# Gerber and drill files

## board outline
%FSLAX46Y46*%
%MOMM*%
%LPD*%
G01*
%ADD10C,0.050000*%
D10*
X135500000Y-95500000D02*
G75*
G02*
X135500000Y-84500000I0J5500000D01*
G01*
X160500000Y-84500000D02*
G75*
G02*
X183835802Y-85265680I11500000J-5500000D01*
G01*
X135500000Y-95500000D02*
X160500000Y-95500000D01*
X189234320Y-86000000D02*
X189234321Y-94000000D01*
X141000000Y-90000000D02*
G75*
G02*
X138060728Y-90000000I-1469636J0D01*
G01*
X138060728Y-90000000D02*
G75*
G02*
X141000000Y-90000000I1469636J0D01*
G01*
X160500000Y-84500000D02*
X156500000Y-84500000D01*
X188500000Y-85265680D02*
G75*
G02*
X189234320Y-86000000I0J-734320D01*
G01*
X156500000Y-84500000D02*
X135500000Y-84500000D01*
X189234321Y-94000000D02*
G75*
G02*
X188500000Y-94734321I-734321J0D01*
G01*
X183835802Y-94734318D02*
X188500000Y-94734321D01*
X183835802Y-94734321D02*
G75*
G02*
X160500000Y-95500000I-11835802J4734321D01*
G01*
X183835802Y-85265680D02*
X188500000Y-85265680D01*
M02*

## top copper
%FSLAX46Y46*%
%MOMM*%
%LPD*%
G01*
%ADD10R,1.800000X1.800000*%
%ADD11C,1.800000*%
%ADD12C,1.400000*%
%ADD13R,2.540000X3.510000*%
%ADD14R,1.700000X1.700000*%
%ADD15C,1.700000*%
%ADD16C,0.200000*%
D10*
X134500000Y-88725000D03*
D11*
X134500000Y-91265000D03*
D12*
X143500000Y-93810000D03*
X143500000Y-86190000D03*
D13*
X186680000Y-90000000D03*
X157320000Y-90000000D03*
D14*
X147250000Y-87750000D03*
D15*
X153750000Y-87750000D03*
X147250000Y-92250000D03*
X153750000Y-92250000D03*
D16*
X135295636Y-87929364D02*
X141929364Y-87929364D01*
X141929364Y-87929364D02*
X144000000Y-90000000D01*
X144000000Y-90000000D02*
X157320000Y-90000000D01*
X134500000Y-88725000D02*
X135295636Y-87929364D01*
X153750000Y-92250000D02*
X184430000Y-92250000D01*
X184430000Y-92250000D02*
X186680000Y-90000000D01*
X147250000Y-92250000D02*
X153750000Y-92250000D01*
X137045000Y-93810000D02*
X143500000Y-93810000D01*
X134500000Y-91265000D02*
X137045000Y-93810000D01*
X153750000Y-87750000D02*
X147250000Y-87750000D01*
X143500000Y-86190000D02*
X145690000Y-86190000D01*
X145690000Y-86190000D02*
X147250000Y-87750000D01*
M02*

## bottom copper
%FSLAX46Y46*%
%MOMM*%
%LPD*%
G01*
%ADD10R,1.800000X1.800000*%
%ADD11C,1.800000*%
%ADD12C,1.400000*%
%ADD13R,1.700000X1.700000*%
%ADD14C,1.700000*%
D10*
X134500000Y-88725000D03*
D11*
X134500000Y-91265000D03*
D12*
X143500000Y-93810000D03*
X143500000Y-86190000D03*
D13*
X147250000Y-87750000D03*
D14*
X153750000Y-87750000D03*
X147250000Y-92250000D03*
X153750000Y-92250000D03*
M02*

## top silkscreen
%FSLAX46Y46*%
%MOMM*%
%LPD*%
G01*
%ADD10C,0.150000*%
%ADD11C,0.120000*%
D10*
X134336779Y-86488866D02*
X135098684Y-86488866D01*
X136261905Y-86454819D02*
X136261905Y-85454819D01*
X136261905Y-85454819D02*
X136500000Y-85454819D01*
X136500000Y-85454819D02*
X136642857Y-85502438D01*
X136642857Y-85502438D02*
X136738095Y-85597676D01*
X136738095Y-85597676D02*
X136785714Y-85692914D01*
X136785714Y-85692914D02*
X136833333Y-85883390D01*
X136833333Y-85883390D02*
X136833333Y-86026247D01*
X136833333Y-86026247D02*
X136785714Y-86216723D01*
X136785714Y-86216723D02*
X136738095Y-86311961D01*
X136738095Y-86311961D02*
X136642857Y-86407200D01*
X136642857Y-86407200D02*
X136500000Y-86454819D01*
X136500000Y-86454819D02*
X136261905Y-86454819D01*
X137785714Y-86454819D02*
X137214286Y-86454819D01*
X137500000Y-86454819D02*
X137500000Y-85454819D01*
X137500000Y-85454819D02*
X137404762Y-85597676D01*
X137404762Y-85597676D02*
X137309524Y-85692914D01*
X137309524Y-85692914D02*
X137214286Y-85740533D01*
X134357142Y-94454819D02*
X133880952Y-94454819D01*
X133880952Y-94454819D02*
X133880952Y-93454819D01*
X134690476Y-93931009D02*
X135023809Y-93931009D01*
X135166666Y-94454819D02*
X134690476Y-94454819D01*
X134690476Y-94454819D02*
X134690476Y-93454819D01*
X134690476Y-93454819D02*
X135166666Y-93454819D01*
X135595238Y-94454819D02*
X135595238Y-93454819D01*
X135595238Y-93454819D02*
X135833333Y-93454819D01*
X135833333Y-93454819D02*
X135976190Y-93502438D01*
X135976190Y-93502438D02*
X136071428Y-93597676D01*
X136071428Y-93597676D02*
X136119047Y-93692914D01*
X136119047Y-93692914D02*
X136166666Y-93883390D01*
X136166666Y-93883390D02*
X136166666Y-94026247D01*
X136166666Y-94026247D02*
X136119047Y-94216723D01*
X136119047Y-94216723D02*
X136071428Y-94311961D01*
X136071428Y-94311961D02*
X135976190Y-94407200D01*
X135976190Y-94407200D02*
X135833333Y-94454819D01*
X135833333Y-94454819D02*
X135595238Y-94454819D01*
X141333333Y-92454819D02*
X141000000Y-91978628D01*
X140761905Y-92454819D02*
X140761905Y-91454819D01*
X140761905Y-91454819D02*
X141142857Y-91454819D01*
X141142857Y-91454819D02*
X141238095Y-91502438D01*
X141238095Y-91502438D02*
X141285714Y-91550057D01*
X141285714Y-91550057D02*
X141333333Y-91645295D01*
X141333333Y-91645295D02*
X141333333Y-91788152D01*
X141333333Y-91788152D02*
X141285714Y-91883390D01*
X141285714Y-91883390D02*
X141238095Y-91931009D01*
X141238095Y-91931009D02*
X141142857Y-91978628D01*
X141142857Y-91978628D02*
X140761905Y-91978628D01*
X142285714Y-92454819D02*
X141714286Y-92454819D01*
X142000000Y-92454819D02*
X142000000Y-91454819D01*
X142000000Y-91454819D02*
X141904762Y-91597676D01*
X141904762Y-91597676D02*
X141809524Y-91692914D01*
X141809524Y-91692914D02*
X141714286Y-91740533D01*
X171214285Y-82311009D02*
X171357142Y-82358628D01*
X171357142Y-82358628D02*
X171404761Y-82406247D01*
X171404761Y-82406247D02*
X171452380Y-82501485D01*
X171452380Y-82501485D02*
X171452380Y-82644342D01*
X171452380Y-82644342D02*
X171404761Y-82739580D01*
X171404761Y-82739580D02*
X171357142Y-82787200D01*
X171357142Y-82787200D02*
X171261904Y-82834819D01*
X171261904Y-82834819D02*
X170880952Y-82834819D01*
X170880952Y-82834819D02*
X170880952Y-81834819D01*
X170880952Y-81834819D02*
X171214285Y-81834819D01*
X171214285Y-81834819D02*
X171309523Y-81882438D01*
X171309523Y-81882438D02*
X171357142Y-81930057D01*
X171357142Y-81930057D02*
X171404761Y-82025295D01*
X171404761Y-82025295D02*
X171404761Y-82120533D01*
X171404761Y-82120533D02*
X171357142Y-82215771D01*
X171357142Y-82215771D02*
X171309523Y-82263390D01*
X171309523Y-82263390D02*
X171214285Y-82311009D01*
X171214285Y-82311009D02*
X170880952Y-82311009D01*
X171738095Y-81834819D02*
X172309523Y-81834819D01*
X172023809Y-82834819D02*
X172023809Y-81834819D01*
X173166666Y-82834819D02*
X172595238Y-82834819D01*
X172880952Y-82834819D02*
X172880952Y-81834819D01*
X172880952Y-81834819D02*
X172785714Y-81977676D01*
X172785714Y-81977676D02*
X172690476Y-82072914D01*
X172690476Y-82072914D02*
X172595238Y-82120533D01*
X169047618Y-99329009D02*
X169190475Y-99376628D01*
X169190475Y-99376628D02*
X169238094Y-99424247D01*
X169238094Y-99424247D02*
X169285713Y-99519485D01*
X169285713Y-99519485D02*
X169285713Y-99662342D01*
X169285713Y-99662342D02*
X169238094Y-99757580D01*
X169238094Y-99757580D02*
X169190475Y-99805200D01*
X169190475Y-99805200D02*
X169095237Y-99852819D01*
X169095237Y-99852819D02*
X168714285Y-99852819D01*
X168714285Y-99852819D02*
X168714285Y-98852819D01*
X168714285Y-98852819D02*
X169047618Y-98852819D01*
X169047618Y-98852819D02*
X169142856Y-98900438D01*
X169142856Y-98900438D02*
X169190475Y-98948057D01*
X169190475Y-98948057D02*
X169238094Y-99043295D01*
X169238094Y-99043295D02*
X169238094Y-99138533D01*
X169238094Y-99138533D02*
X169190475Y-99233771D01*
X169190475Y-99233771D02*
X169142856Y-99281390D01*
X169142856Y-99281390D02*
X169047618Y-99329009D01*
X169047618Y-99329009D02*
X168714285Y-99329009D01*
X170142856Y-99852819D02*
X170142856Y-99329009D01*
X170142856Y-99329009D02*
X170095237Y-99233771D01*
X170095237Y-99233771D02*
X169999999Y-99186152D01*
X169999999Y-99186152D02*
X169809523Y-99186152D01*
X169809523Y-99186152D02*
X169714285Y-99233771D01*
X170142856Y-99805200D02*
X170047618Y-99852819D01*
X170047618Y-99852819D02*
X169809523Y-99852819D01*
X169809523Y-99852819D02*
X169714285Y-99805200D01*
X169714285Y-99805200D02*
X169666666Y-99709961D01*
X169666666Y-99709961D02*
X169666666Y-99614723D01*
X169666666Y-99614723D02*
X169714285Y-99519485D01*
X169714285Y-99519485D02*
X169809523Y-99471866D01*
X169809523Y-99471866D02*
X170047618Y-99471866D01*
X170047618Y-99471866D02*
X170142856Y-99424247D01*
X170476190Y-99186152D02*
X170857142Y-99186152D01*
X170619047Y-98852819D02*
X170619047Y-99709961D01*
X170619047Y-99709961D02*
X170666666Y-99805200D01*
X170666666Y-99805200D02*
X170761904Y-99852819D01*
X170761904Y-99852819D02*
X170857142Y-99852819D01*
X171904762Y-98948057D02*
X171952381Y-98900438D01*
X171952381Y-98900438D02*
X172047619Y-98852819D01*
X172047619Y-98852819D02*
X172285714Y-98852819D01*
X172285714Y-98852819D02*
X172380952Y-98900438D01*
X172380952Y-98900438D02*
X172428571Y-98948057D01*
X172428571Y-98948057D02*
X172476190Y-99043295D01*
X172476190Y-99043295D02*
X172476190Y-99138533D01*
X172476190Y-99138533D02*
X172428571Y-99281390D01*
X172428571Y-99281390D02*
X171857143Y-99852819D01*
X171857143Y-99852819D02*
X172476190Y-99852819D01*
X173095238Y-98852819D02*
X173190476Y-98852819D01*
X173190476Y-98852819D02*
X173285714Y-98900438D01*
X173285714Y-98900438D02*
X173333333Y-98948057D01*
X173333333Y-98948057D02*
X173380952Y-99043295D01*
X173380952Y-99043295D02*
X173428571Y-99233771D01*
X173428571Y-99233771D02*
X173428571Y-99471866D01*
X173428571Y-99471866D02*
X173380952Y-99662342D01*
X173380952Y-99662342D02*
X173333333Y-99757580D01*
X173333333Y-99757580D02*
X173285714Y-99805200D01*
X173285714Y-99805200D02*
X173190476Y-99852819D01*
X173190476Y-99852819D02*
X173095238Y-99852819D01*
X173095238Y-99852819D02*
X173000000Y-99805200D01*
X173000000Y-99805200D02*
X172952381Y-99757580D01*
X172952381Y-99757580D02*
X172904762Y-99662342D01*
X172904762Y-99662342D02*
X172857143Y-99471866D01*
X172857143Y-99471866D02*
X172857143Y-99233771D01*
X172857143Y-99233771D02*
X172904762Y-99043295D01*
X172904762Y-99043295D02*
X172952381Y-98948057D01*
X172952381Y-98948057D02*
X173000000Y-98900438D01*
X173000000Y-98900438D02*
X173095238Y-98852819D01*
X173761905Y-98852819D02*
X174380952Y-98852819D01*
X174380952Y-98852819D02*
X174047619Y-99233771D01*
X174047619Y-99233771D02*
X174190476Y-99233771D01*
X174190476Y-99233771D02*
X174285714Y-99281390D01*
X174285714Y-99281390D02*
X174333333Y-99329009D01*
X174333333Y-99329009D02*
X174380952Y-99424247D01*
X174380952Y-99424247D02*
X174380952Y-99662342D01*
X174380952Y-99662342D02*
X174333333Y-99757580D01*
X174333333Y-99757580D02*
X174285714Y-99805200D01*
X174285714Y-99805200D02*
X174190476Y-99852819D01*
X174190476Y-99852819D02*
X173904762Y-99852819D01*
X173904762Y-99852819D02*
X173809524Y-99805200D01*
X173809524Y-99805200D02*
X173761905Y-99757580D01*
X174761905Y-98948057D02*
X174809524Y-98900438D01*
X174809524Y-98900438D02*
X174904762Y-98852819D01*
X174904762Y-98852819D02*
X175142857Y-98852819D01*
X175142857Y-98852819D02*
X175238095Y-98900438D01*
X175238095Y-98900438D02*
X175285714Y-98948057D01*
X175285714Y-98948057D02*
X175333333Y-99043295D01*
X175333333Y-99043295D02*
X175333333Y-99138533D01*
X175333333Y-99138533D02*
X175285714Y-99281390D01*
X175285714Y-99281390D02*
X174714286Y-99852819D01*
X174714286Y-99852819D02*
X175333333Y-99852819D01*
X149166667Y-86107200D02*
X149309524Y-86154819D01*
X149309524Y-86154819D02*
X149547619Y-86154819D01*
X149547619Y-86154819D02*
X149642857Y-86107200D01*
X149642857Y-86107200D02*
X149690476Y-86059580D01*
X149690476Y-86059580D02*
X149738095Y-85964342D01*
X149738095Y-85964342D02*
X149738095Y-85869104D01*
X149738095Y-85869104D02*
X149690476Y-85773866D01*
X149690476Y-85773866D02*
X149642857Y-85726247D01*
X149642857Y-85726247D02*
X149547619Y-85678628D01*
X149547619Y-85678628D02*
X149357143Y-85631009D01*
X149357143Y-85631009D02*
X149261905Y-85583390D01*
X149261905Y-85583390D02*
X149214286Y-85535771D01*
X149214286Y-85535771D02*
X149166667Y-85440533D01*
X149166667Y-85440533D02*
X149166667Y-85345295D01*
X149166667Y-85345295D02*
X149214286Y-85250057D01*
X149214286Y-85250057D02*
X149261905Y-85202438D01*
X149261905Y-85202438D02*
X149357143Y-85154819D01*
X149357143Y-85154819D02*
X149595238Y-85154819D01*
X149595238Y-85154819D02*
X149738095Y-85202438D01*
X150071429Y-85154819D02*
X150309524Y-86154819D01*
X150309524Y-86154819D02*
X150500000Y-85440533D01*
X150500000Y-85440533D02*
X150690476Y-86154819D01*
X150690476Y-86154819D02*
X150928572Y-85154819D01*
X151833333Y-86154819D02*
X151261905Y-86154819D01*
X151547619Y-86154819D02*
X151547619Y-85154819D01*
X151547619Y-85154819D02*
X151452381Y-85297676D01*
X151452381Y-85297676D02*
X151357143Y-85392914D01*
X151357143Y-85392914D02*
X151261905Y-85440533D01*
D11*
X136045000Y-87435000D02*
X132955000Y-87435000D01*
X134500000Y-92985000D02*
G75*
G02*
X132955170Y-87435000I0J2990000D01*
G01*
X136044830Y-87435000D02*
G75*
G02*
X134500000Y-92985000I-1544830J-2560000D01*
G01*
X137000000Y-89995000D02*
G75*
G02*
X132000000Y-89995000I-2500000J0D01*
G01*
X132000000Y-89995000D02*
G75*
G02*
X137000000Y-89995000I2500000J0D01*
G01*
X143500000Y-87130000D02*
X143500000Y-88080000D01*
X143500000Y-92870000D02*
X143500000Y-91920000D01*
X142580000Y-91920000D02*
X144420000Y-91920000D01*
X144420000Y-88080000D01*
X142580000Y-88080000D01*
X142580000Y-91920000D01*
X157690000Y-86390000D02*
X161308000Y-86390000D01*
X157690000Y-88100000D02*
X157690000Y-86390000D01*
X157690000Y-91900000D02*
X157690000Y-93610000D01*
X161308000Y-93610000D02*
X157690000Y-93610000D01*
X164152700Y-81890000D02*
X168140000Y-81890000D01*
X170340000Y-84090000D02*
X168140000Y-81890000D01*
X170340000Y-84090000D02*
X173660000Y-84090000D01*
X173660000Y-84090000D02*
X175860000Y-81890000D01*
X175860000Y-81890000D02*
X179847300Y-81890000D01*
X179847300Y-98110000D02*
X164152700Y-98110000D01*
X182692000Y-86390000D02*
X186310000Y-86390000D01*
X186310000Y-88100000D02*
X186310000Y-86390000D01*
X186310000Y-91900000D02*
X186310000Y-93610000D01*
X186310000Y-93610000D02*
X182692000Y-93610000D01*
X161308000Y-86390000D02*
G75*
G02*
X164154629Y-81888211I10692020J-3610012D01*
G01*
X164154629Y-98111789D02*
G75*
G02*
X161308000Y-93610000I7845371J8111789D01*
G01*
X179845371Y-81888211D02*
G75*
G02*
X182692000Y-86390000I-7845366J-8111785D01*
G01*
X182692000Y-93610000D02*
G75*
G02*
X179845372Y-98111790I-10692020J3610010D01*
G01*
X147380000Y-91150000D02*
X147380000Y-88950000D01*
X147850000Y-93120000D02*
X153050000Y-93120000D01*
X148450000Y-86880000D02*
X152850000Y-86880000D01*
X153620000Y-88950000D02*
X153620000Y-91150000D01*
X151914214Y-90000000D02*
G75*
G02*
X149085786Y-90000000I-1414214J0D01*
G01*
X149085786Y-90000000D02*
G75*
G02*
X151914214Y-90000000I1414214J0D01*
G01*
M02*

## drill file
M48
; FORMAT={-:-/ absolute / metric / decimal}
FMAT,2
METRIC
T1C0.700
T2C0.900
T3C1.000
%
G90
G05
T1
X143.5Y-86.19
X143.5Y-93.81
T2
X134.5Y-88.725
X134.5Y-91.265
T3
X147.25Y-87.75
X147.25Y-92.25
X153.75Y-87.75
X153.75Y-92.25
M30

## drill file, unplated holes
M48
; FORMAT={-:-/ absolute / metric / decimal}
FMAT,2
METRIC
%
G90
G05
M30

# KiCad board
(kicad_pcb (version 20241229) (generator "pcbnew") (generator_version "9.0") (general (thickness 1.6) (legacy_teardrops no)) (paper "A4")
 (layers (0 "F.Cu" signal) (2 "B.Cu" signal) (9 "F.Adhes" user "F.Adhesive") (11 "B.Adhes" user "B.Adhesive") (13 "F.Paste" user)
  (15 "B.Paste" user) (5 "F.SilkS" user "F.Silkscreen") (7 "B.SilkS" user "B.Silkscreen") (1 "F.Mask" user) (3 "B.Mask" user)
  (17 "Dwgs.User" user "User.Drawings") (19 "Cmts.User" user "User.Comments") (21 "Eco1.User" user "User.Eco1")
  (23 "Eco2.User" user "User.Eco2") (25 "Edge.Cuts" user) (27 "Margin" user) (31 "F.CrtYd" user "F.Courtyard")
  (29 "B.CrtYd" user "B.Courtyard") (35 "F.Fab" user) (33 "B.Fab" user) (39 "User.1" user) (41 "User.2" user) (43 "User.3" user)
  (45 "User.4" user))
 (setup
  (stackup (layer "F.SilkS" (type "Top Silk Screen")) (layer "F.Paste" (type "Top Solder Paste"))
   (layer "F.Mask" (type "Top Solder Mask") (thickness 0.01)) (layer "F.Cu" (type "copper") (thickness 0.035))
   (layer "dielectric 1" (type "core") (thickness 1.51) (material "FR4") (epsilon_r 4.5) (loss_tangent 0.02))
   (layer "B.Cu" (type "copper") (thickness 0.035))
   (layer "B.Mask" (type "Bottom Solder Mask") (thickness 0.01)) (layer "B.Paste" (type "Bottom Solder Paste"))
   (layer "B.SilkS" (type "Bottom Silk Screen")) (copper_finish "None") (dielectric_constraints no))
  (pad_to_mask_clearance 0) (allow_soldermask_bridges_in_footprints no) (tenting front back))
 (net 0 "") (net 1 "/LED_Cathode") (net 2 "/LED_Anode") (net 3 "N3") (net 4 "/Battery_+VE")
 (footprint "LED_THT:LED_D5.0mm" (layer "F.Cu") (at 134.5 88.725 -90)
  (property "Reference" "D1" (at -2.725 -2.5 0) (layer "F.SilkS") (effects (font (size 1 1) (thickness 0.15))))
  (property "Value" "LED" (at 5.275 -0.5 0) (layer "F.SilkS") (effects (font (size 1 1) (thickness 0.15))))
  (fp_line (start -1.29 -1.545) (end -1.29 1.545) (stroke (width 0.12) (type solid)) (layer "F.SilkS"))
  (fp_arc (start 4.26 0) (mid 2.071779 2.880495) (end -1.29 1.54483) (stroke (width 0.12) (type solid)) (layer "F.SilkS"))
  (fp_arc (start -1.29 -1.54483) (mid 2.071779 -2.880495) (end 4.26 0) (stroke (width 0.12) (type solid)) (layer "F.SilkS"))
  (fp_circle (center 1.27 0) (end 3.77 0) (stroke (width 0.12) (type solid)) (fill no) (layer "F.SilkS"))
  (pad "1" thru_hole rect (at 0 0 270) (size 1.8 1.8) (drill 0.9) (layers "*.Cu" "*.Mask") (remove_unused_layers no) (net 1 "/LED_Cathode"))
  (pad "2" thru_hole circle (at 2.54 0 270) (size 1.8 1.8) (drill 0.9) (layers "*.Cu" "*.Mask") (remove_unused_layers no)
   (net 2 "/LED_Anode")))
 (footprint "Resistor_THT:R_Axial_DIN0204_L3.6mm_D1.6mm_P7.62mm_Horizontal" (layer "F.Cu") (at 143.5 93.81 90)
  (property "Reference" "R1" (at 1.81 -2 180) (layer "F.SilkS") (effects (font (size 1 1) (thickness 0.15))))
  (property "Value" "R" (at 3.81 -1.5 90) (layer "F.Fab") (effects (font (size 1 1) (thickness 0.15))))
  (fp_line (start 6.68 0) (end 5.73 0) (stroke (width 0.12) (type solid)) (layer "F.SilkS"))
  (fp_line (start 0.94 0) (end 1.89 0) (stroke (width 0.12) (type solid)) (layer "F.SilkS"))
  (fp_rect (start 1.89 -0.92) (end 5.73 0.92) (stroke (width 0.12) (type solid)) (fill no) (layer "F.SilkS"))
  (pad "1" thru_hole circle (at 0 0 90) (size 1.4 1.4) (drill 0.7) (layers "*.Cu" "*.Mask") (remove_unused_layers no) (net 2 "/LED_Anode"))
  (pad "2" thru_hole circle (at 7.62 0 90) (size 1.4 1.4) (drill 0.7) (layers "*.Cu" "*.Mask") (remove_unused_layers no) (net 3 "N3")))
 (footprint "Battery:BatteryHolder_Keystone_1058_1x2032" (layer "F.Cu") (at 172 90 180)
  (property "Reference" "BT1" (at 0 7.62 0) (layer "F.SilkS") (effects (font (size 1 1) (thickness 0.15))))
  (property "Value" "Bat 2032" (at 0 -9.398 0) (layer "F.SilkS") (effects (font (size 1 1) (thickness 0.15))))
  (fp_line (start 14.31 3.61) (end 10.692 3.61) (stroke (width 0.12) (type solid)) (layer "F.SilkS"))
  (fp_line (start 14.31 1.9) (end 14.31 3.61) (stroke (width 0.12) (type solid)) (layer "F.SilkS"))
  (fp_line (start 14.31 -1.9) (end 14.31 -3.61) (stroke (width 0.12) (type solid)) (layer "F.SilkS"))
  (fp_line (start 10.692 -3.61) (end 14.31 -3.61) (stroke (width 0.12) (type solid)) (layer "F.SilkS"))
  (fp_line (start 7.8473 8.11) (end 3.86 8.11) (stroke (width 0.12) (type solid)) (layer "F.SilkS"))
  (fp_line (start 1.66 5.91) (end 3.86 8.11) (stroke (width 0.12) (type solid)) (layer "F.SilkS"))
  (fp_line (start 1.66 5.91) (end -1.66 5.91) (stroke (width 0.12) (type solid)) (layer "F.SilkS"))
  (fp_line (start -1.66 5.91) (end -3.86 8.11) (stroke (width 0.12) (type solid)) (layer "F.SilkS"))
  (fp_line (start -3.86 8.11) (end -7.8473 8.11) (stroke (width 0.12) (type solid)) (layer "F.SilkS"))
  (fp_line (start -7.8473 -8.11) (end 7.8473 -8.11) (stroke (width 0.12) (type solid)) (layer "F.SilkS"))
  (fp_line (start -10.692 3.61) (end -14.31 3.61) (stroke (width 0.12) (type solid)) (layer "F.SilkS"))
  (fp_line (start -14.31 1.9) (end -14.31 3.61) (stroke (width 0.12) (type solid)) (layer "F.SilkS"))
  (fp_line (start -14.31 -1.9) (end -14.31 -3.61) (stroke (width 0.12) (type solid)) (layer "F.SilkS"))
  (fp_line (start -14.31 -3.61) (end -10.692 -3.61) (stroke (width 0.12) (type solid)) (layer "F.SilkS"))
  (fp_arc (start 10.692 3.61) (mid 9.538084 6.031244) (end 7.845371 8.111789) (stroke (width 0.12) (type solid)) (layer "F.SilkS"))
  (fp_arc (start 7.845371 -8.111789) (mid 9.538085 -6.031244) (end 10.692 -3.61) (stroke (width 0.12) (type solid)) (layer "F.SilkS"))
  (fp_arc (start -7.845371 8.111789) (mid -9.538085 6.031244) (end -10.692 3.61) (stroke (width 0.12) (type solid)) (layer "F.SilkS"))
  (fp_arc (start -10.692 -3.61) (mid -9.538084 -6.031244) (end -7.845371 -8.111789) (stroke (width 0.12) (type solid)) (layer "F.SilkS"))
  (pad "1" smd rect (at -14.68 0 180) (size 2.54 3.51) (layers "F.Cu" "F.Mask" "F.Paste") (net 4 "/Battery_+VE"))
  (pad "2" smd rect (at 14.68 0 180) (size 2.54 3.51) (layers "F.Cu" "F.Mask" "F.Paste") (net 1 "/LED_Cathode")))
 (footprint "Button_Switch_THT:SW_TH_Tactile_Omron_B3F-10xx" (layer "F.Cu") (at 147.25 87.75)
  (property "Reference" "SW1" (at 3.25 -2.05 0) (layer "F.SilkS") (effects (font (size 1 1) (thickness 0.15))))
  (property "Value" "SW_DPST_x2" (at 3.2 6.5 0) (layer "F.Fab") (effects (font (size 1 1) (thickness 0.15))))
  (fp_line (start 0.13 3.4) (end 0.13 1.2) (stroke (width 0.12) (type solid)) (layer "F.SilkS"))
  (fp_line (start 0.6 5.37) (end 5.8 5.37) (stroke (width 0.12) (type solid)) (layer "F.SilkS"))
  (fp_line (start 1.2 -0.87) (end 5.6 -0.87) (stroke (width 0.12) (type solid)) (layer "F.SilkS"))
  (fp_line (start 6.37 1.2) (end 6.37 3.4) (stroke (width 0.12) (type solid)) (layer "F.SilkS"))
  (fp_circle (center 3.25 2.25) (end 4.25 3.25) (stroke (width 0.12) (type solid)) (fill no) (layer "F.SilkS"))
  (pad "1" thru_hole rect (at 0 0) (size 1.7 1.7) (drill 1) (layers "*.Cu" "*.Mask") (remove_unused_layers no) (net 3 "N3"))
  (pad "1" thru_hole circle (at 6.5 0) (size 1.7 1.7) (drill 1) (layers "*.Cu" "*.Mask") (remove_unused_layers no) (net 3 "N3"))
  (pad "2" thru_hole circle (at 0 4.5) (size 1.7 1.7) (drill 1) (layers "*.Cu" "*.Mask") (remove_unused_layers no) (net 4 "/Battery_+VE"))
  (pad "2" thru_hole circle (at 6.5 4.5) (size 1.7 1.7) (drill 1) (layers "*.Cu" "*.Mask") (remove_unused_layers no) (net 4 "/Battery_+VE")))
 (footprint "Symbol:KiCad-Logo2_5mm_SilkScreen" (layer "B.Cu") (at 172 89 180)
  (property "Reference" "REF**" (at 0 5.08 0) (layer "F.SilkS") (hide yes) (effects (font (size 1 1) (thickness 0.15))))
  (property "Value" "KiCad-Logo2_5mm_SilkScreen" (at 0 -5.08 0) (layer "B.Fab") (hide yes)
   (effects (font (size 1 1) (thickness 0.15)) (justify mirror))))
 (gr_arc (start 135.5 95.5) (mid 130 90) (end 135.5 84.5) (stroke (width 0.05) (type default)) (locked yes) (layer "Edge.Cuts"))
 (gr_arc (start 160.5 84.5) (mid 172.41804 77.259308) (end 183.835802 85.26568) (stroke (width 0.05) (type default)) (locked yes)
  (layer "Edge.Cuts"))
 (gr_line (start 135.5 95.5) (end 160.5 95.5) (stroke (width 0.05) (type default)) (locked yes) (layer "Edge.Cuts"))
 (gr_line (start 189.23432 86) (end 189.234321 94) (stroke (width 0.05) (type default)) (locked yes) (layer "Edge.Cuts"))
 (gr_circle (center 139.530364 90) (end 138.148398 89.5) (stroke (width 0.05) (type default)) (fill no) (layer "Edge.Cuts"))
 (gr_line (start 160.5 84.5) (end 156.5 84.5) (stroke (width 0.05) (type default)) (locked yes) (layer "Edge.Cuts"))
 (gr_arc (start 188.5 85.26568) (mid 189.019243 85.480757) (end 189.23432 86) (stroke (width 0.05) (type default)) (locked yes)
  (layer "Edge.Cuts"))
 (gr_line (start 156.5 84.5) (end 135.5 84.5) (stroke (width 0.05) (type default)) (locked yes) (layer "Edge.Cuts"))
 (gr_arc (start 189.234321 94) (mid 189.019243 94.519243) (end 188.5 94.734321) (stroke (width 0.05) (type default)) (locked yes)
  (layer "Edge.Cuts"))
 (gr_line (start 183.835802 94.734318) (end 188.5 94.734321) (stroke (width 0.05) (type default)) (locked yes) (layer "Edge.Cuts"))
 (gr_arc (start 183.835802 94.734321) (mid 172.418039 102.740693) (end 160.5 95.5) (stroke (width 0.05) (type default)) (locked yes)
  (layer "Edge.Cuts"))
 (gr_line (start 183.835802 85.26568) (end 188.5 85.26568) (stroke (width 0.05) (type default)) (locked yes) (layer "Edge.Cuts"))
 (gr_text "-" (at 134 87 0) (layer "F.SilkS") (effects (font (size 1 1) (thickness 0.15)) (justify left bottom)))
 (segment (start 135.295636 87.929364) (end 141.929364 87.929364) (width 0.2) (layer "F.Cu") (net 1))
 (segment (start 141.929364 87.929364) (end 144 90) (width 0.2) (layer "F.Cu") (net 1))
 (segment (start 144 90) (end 157.32 90) (width 0.2) (layer "F.Cu") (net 1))
 (segment (start 134.5 88.725) (end 135.295636 87.929364) (width 0.2) (layer "F.Cu") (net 1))
 (segment (start 153.75 92.25) (end 184.43 92.25) (width 0.2) (layer "F.Cu") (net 4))
 (segment (start 184.43 92.25) (end 186.68 90) (width 0.2) (layer "F.Cu") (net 4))
 (segment (start 147.25 92.25) (end 153.75 92.25) (width 0.2) (layer "F.Cu") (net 4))
 (segment (start 137.045 93.81) (end 143.5 93.81) (width 0.2) (layer "F.Cu") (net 2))
 (segment (start 134.5 91.265) (end 137.045 93.81) (width 0.2) (layer "F.Cu") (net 2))
 (segment (start 153.75 87.75) (end 147.25 87.75) (width 0.2) (layer "F.Cu") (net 3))
 (segment (start 143.5 86.19) (end 145.69 86.19) (width 0.2) (layer "F.Cu") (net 3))
 (segment (start 145.69 86.19) (end 147.25 87.75) (width 0.2) (layer "F.Cu") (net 3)))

